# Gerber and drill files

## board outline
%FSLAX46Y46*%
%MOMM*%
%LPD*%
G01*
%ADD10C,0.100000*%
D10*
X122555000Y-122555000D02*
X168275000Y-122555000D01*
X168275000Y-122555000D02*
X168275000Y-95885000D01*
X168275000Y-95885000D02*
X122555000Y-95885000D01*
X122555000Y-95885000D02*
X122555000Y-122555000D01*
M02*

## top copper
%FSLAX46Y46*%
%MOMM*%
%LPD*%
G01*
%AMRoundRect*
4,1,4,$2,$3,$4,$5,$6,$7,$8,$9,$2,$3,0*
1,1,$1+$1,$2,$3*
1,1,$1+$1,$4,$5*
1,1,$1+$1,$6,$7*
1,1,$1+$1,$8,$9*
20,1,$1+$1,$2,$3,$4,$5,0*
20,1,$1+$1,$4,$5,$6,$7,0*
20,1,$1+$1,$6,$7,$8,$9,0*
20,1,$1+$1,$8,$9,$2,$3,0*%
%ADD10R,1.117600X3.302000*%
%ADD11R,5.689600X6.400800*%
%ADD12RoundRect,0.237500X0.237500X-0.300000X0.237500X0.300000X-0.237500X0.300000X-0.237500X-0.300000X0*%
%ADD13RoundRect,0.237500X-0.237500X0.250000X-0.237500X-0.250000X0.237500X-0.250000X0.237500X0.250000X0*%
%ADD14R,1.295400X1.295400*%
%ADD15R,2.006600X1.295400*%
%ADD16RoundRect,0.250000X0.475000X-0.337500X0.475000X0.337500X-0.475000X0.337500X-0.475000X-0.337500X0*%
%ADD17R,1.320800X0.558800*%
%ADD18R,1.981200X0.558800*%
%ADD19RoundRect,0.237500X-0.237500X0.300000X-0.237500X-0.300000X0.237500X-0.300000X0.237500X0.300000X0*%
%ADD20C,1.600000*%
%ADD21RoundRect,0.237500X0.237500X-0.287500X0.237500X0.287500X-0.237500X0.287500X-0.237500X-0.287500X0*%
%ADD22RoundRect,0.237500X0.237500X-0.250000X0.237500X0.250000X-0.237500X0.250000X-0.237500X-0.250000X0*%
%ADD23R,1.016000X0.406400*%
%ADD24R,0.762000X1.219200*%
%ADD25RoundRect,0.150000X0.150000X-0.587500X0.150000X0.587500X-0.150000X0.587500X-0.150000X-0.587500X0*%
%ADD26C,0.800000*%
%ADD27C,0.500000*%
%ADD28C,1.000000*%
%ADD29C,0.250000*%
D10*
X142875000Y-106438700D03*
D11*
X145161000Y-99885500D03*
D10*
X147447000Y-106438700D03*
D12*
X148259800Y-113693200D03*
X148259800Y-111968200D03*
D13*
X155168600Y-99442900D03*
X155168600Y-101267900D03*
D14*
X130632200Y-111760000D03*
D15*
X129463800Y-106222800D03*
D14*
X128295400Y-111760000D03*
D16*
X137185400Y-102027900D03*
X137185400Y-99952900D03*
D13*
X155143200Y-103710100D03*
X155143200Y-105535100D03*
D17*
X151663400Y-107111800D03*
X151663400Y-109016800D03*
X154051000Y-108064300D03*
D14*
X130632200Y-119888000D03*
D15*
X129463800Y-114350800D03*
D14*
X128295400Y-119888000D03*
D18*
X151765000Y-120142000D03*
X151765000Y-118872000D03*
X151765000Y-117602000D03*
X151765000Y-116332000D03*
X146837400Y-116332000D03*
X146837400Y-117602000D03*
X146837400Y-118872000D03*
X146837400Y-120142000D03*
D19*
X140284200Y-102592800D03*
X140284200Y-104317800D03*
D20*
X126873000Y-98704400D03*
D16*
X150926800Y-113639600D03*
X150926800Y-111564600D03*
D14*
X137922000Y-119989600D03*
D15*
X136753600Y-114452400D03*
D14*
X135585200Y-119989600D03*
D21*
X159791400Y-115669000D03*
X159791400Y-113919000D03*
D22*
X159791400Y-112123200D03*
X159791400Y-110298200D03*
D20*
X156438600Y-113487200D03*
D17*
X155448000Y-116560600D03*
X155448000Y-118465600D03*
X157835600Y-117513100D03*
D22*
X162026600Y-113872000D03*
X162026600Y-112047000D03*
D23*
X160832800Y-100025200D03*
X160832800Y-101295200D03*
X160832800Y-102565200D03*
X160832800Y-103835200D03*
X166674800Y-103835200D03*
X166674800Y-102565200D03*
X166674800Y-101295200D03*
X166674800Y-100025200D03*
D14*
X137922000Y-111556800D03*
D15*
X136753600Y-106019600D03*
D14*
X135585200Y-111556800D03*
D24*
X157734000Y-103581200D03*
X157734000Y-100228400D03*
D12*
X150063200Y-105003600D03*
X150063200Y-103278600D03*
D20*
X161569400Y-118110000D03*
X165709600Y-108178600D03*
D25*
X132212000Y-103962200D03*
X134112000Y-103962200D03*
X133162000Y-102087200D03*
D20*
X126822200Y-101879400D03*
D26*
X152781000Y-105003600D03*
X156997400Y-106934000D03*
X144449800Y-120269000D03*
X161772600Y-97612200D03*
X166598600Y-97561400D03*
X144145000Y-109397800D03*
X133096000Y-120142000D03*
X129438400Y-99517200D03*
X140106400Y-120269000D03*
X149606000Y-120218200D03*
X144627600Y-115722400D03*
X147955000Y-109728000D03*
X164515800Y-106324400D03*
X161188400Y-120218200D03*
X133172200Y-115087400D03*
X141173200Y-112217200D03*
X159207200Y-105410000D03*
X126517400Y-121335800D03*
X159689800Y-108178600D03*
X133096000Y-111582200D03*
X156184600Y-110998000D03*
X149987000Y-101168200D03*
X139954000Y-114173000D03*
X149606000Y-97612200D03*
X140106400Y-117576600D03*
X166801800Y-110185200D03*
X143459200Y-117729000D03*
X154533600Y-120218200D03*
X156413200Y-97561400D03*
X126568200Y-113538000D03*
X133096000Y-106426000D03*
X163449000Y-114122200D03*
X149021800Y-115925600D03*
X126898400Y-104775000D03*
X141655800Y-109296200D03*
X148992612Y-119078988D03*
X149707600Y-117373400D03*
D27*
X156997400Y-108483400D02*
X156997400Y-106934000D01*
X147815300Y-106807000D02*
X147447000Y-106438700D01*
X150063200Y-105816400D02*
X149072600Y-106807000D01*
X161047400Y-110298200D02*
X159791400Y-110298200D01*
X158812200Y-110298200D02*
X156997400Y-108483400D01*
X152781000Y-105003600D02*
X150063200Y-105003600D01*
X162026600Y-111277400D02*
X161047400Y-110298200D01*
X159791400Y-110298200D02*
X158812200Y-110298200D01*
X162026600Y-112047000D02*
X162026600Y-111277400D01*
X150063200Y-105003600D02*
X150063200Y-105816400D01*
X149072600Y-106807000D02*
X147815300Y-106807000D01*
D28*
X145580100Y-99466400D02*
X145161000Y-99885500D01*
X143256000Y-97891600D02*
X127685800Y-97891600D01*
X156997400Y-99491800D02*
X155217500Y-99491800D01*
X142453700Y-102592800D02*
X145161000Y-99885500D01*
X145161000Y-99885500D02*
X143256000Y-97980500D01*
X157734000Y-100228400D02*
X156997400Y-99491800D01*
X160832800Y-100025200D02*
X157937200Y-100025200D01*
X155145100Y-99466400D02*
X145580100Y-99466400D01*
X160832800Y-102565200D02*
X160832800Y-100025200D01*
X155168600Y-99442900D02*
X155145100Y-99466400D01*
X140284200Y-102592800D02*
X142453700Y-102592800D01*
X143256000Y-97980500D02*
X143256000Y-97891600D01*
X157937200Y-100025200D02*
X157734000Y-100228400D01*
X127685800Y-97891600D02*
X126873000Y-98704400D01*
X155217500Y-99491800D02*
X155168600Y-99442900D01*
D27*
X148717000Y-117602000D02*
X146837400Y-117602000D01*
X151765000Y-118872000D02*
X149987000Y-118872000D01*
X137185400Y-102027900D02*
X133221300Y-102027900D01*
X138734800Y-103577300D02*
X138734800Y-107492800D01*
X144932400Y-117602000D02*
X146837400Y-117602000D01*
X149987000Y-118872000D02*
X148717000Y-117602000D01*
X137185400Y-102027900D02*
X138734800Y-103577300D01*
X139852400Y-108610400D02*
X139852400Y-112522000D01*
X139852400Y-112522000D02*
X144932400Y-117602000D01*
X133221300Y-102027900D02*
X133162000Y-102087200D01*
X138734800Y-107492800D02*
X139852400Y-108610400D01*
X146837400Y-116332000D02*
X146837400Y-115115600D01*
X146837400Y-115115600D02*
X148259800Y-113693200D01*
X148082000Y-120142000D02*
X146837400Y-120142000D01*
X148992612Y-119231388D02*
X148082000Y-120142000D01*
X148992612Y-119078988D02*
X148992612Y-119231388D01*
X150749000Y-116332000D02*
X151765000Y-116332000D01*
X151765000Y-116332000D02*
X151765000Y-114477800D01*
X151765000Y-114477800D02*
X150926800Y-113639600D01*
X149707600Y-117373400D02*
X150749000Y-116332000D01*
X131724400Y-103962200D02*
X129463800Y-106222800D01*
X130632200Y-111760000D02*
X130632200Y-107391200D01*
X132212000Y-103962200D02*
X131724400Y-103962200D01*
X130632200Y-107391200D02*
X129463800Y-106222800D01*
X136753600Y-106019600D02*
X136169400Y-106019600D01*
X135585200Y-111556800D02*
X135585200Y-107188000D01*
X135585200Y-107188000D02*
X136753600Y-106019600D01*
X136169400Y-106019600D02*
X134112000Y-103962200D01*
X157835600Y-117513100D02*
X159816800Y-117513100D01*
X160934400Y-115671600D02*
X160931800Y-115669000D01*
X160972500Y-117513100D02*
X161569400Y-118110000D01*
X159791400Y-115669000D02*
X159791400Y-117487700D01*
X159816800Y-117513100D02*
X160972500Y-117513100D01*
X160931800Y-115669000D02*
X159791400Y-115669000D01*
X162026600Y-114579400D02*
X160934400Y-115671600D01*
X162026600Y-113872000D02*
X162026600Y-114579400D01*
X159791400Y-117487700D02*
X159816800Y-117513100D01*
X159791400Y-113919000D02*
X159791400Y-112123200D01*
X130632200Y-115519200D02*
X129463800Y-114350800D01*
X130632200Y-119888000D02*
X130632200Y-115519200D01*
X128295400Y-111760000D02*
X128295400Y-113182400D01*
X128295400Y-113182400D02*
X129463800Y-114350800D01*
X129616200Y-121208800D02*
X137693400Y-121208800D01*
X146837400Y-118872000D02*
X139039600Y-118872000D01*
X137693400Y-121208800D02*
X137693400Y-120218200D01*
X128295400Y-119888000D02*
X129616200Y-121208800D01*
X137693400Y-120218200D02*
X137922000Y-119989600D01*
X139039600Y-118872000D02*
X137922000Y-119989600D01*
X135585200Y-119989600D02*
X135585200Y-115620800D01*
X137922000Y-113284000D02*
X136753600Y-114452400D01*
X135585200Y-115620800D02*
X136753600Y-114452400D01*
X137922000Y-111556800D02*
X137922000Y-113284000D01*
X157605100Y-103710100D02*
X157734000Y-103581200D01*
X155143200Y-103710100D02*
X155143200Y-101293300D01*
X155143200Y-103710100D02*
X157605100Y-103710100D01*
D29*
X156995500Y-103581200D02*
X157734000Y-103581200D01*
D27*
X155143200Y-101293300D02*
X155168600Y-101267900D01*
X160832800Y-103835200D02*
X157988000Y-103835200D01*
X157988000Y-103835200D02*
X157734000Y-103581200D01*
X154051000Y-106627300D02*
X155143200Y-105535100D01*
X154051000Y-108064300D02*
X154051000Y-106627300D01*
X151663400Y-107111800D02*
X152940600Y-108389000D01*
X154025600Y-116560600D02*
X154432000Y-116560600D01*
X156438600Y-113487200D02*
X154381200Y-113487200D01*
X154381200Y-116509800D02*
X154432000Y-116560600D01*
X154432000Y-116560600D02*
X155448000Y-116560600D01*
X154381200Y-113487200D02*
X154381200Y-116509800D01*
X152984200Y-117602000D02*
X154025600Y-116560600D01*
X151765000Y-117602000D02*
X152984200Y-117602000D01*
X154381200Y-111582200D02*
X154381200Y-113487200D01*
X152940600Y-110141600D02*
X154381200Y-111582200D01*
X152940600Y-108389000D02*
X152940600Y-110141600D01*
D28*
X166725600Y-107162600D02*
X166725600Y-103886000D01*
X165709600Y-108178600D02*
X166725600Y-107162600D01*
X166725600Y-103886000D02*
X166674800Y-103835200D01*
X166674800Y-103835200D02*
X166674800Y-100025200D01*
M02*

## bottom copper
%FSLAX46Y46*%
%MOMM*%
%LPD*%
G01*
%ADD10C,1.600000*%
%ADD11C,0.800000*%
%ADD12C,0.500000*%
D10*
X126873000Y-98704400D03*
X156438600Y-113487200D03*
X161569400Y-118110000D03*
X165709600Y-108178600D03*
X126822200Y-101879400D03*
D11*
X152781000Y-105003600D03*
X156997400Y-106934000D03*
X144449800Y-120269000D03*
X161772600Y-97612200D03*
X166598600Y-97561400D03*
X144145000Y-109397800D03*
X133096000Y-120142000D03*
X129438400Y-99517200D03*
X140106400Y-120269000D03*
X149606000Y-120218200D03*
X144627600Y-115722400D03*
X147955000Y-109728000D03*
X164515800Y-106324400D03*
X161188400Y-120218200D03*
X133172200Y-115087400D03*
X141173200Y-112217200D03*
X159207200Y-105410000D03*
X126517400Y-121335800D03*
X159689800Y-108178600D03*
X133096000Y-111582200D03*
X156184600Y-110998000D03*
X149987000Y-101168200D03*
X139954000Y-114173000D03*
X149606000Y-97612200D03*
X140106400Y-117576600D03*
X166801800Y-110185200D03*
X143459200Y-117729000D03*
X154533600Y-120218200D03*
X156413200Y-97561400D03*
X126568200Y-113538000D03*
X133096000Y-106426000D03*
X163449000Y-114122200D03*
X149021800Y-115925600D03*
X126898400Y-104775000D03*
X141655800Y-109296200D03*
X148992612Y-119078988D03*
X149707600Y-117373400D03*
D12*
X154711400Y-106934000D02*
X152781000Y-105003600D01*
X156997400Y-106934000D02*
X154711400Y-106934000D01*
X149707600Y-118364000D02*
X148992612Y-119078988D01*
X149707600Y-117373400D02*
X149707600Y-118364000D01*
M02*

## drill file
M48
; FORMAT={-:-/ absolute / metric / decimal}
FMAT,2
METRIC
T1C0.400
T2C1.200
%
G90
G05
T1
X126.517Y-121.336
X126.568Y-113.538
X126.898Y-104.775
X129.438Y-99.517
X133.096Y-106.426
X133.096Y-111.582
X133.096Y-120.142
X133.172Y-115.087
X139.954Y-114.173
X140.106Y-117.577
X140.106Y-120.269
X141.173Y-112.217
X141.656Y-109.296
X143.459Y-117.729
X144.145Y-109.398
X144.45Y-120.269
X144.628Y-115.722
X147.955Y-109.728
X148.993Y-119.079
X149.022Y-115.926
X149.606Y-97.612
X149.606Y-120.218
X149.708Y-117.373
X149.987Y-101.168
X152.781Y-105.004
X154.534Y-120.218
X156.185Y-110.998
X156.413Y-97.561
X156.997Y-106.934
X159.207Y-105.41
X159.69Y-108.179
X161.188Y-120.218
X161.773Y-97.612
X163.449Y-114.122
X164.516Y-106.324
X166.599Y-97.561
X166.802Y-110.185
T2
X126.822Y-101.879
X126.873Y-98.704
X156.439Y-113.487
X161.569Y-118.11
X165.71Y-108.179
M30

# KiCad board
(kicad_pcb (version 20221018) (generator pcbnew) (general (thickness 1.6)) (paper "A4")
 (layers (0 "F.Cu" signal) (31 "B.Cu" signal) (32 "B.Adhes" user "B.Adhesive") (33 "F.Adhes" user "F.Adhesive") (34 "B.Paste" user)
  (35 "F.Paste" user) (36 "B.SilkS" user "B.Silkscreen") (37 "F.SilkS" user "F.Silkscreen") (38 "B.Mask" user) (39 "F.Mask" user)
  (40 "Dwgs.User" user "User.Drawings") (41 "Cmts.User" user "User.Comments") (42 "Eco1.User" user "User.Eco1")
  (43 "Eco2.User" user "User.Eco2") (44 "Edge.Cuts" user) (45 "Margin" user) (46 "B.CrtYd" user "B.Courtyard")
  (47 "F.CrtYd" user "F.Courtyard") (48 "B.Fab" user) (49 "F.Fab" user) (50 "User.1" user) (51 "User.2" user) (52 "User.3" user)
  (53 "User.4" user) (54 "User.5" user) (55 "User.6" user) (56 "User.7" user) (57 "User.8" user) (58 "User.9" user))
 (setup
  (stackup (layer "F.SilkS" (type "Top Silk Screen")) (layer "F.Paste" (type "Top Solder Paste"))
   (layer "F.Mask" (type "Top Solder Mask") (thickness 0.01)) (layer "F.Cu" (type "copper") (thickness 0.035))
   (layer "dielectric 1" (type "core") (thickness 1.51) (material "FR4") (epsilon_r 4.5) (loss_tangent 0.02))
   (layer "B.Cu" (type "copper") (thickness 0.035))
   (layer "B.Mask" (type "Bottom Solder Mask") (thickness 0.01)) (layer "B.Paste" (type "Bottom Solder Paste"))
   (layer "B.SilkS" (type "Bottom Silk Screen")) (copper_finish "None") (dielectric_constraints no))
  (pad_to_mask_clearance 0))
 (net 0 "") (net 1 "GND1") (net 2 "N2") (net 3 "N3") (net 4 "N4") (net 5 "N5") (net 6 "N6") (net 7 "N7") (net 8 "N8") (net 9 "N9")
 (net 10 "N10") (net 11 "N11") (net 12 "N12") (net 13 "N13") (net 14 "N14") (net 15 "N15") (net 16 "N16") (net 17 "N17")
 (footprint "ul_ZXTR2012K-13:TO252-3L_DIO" (layer "F.Cu") (at 145.161 99.8855)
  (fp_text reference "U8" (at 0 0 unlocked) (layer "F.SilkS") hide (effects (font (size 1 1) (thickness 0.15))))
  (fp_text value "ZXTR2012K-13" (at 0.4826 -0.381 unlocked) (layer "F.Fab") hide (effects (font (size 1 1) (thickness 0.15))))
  (pad "1" smd rect (at -2.286 6.5532) (size 1.1176 3.302) (layers "F.Cu" "F.Paste" "F.Mask") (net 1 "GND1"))
  (pad "2" smd rect (at 0 0) (size 5.6896 6.4008) (layers "F.Cu" "F.Paste" "F.Mask") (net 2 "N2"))
  (pad "3" smd rect (at 2.286 6.5532) (size 1.1176 3.302) (layers "F.Cu" "F.Paste" "F.Mask") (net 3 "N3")))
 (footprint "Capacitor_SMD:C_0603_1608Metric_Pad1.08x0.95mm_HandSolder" (layer "F.Cu") (at 148.2598 112.8307 90)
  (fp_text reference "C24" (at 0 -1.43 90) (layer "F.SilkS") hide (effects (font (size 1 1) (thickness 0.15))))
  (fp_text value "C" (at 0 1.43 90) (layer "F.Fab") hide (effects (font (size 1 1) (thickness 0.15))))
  (pad "1" smd roundrect (at -0.8625 0 90) (size 1.075 0.95) (layers "F.Cu" "F.Paste" "F.Mask") (roundrect_rratio 0.25) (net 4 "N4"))
  (pad "2" smd roundrect (at 0.8625 0 90) (size 1.075 0.95) (layers "F.Cu" "F.Paste" "F.Mask") (roundrect_rratio 0.25) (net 1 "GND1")))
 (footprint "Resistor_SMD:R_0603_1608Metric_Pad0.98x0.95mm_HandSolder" (layer "F.Cu") (at 155.1686 100.3554 -90)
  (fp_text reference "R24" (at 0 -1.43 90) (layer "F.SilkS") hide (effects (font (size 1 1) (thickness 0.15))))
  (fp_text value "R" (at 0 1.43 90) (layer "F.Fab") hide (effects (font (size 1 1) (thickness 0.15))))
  (pad "1" smd roundrect (at -0.9125 0 270) (size 0.975 0.95) (layers "F.Cu" "F.Paste" "F.Mask") (roundrect_rratio 0.25) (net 2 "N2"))
  (pad "2" smd roundrect (at 0.9125 0 270) (size 0.975 0.95) (layers "F.Cu" "F.Paste" "F.Mask") (roundrect_rratio 0.25) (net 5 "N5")))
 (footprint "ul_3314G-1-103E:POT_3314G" (layer "F.Cu") (at 129.4638 108.9914)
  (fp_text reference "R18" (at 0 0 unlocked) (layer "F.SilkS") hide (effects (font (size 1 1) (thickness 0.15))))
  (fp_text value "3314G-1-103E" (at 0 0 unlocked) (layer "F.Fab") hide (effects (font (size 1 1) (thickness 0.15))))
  (pad "1" smd rect (at 1.1684 2.7686) (size 1.2954 1.2954) (layers "F.Cu" "F.Paste" "F.Mask") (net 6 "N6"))
  (pad "2" smd rect (at 0 -2.7686) (size 2.0066 1.2954) (layers "F.Cu" "F.Paste" "F.Mask") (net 6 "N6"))
  (pad "3" smd rect (at -1.1684 2.7686) (size 1.2954 1.2954) (layers "F.Cu" "F.Paste" "F.Mask") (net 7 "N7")))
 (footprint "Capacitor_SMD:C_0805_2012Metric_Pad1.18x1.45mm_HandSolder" (layer "F.Cu") (at 137.1854 100.9904 90)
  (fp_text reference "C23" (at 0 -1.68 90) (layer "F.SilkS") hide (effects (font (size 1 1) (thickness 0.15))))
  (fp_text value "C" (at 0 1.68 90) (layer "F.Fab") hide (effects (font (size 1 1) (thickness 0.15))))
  (pad "1" smd roundrect (at -1.0375 0 90) (size 1.175 1.45) (layers "F.Cu" "F.Paste" "F.Mask") (roundrect_rratio 0.212766) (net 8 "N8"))
  (pad "2" smd roundrect (at 1.0375 0 90) (size 1.175 1.45) (layers "F.Cu" "F.Paste" "F.Mask") (roundrect_rratio 0.212766) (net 1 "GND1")))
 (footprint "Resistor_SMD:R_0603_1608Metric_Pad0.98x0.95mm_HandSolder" (layer "F.Cu") (at 155.1432 104.6226 -90)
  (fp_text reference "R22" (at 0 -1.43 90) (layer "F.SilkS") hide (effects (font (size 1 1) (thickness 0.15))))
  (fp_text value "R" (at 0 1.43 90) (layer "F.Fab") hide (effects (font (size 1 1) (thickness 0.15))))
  (pad "1" smd roundrect (at -0.9125 0 270) (size 0.975 0.95) (layers "F.Cu" "F.Paste" "F.Mask") (roundrect_rratio 0.25) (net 5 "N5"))
  (pad "2" smd roundrect (at 0.9125 0 270) (size 0.975 0.95) (layers "F.Cu" "F.Paste" "F.Mask") (roundrect_rratio 0.25) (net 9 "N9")))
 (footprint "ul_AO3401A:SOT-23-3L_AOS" (layer "F.Cu") (at 152.8572 108.0643 -90)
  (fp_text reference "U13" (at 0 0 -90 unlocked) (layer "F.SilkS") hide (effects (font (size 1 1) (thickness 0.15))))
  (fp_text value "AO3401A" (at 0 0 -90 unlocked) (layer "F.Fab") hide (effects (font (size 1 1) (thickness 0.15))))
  (pad "1" smd rect (at -0.9525 1.1938 270) (size 0.5588 1.3208) (layers "F.Cu" "F.Paste" "F.Mask") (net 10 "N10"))
  (pad "2" smd rect (at 0.9525 1.1938 270) (size 0.5588 1.3208) (layers "F.Cu" "F.Paste" "F.Mask") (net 1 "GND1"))
  (pad "3" smd rect (at 0 -1.1938 270) (size 0.5588 1.3208) (layers "F.Cu" "F.Paste" "F.Mask") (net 9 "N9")))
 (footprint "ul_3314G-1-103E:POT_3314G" (layer "F.Cu") (at 129.4638 117.1194)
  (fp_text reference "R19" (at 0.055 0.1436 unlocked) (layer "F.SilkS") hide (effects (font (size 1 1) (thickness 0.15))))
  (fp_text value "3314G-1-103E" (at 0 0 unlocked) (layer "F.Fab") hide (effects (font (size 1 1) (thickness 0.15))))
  (pad "1" smd rect (at 1.1684 2.7686) (size 1.2954 1.2954) (layers "F.Cu" "F.Paste" "F.Mask") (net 7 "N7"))
  (pad "2" smd rect (at 0 -2.7686) (size 2.0066 1.2954) (layers "F.Cu" "F.Paste" "F.Mask") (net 7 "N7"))
  (pad "3" smd rect (at -1.1684 2.7686) (size 1.2954 1.2954) (layers "F.Cu" "F.Paste" "F.Mask") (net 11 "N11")))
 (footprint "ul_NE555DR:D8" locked (layer "F.Cu") (at 149.3012 118.237 180)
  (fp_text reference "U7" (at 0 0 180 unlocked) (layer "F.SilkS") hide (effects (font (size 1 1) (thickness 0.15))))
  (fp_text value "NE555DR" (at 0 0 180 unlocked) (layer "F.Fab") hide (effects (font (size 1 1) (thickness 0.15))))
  (pad "1" smd rect locked (at -2.4638 -1.905 180) (size 1.9812 0.5588) (layers "F.Cu" "F.Paste" "F.Mask") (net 1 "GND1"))
  (pad "2" smd rect locked (at -2.4638 -0.635 180) (size 1.9812 0.5588) (layers "F.Cu" "F.Paste" "F.Mask") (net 8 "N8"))
  (pad "3" smd rect locked (at -2.4638 0.635 180) (size 1.9812 0.5588) (layers "F.Cu" "F.Paste" "F.Mask") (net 10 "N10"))
  (pad "4" smd rect locked (at -2.4638 1.905 180) (size 1.9812 0.5588) (layers "F.Cu" "F.Paste" "F.Mask") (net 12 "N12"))
  (pad "5" smd rect locked (at 2.4638 1.905 180) (size 1.9812 0.5588) (layers "F.Cu" "F.Paste" "F.Mask") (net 4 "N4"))
  (pad "6" smd rect locked (at 2.4638 0.635 180) (size 1.9812 0.5588) (layers "F.Cu" "F.Paste" "F.Mask") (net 8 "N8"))
  (pad "7" smd rect locked (at 2.4638 -0.635 180) (size 1.9812 0.5588) (layers "F.Cu" "F.Paste" "F.Mask") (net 11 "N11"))
  (pad "8" smd rect locked (at 2.4638 -1.905 180) (size 1.9812 0.5588) (layers "F.Cu" "F.Paste" "F.Mask") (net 12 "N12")))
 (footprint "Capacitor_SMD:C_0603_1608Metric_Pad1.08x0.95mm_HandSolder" (layer "F.Cu") (at 140.2842 103.4553 -90)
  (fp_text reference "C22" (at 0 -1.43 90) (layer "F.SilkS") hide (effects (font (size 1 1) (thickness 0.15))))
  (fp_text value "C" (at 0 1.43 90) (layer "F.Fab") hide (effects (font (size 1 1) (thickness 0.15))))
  (pad "1" smd roundrect (at -0.8625 0 270) (size 1.075 0.95) (layers "F.Cu" "F.Paste" "F.Mask") (roundrect_rratio 0.25) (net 2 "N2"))
  (pad "2" smd roundrect (at 0.8625 0 270) (size 1.075 0.95) (layers "F.Cu" "F.Paste" "F.Mask") (roundrect_rratio 0.25) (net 1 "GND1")))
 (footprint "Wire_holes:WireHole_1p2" (layer "F.Cu") (at 126.873 98.7044)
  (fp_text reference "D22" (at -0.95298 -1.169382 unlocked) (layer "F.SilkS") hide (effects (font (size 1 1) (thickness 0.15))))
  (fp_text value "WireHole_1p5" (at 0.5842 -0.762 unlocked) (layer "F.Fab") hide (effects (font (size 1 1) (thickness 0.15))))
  (pad "1" thru_hole circle (at 0 0) (size 1.6 1.6) (drill 1.2) (layers "*.Cu" "*.Mask") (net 2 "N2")))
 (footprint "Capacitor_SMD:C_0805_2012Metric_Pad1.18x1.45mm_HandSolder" (layer "F.Cu") (at 150.9268 112.6021 90)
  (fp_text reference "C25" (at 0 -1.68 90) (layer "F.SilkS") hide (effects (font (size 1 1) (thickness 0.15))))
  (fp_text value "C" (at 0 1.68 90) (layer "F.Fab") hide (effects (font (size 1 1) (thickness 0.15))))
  (pad "1" smd roundrect (at -1.0375 0 90) (size 1.175 1.45) (layers "F.Cu" "F.Paste" "F.Mask") (roundrect_rratio 0.212766) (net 12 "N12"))
  (pad "2" smd roundrect (at 1.0375 0 90) (size 1.175 1.45) (layers "F.Cu" "F.Paste" "F.Mask") (roundrect_rratio 0.212766) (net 1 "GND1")))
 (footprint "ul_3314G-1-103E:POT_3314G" (layer "F.Cu") (at 136.7536 117.221)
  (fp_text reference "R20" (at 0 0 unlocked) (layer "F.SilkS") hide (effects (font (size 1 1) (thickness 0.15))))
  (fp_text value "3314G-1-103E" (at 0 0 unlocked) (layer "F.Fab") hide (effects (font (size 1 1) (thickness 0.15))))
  (pad "1" smd rect (at 1.1684 2.7686) (size 1.2954 1.2954) (layers "F.Cu" "F.Paste" "F.Mask") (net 11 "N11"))
  (pad "2" smd rect (at 0 -2.7686) (size 2.0066 1.2954) (layers "F.Cu" "F.Paste" "F.Mask") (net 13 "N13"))
  (pad "3" smd rect (at -1.1684 2.7686) (size 1.2954 1.2954) (layers "F.Cu" "F.Paste" "F.Mask") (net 13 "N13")))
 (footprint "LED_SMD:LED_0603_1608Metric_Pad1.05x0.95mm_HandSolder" (layer "F.Cu") (at 159.7914 114.794 90)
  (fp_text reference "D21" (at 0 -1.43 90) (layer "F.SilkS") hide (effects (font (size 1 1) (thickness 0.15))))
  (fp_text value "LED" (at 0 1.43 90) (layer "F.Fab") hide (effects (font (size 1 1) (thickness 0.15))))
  (pad "1" smd roundrect (at -0.875 0 90) (size 1.05 0.95) (layers "F.Cu" "F.Paste" "F.Mask") (roundrect_rratio 0.25) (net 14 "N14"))
  (pad "2" smd roundrect (at 0.875 0 90) (size 1.05 0.95) (layers "F.Cu" "F.Paste" "F.Mask") (roundrect_rratio 0.25) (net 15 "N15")))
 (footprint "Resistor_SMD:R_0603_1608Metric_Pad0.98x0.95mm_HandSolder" (layer "F.Cu") (at 159.7914 111.2107 90)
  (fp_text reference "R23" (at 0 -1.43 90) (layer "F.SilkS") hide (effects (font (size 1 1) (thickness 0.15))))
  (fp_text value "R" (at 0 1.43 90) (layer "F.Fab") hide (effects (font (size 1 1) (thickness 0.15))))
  (pad "1" smd roundrect (at -0.9125 0 90) (size 0.975 0.95) (layers "F.Cu" "F.Paste" "F.Mask") (roundrect_rratio 0.25) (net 15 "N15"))
  (pad "2" smd roundrect (at 0.9125 0 90) (size 0.975 0.95) (layers "F.Cu" "F.Paste" "F.Mask") (roundrect_rratio 0.25) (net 3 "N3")))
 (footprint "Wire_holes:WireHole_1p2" (layer "F.Cu") (at 156.4386 113.4872)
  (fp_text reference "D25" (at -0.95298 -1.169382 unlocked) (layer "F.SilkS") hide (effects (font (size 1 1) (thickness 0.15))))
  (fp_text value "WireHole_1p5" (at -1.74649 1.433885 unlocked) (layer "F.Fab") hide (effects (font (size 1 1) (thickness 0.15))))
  (pad "1" thru_hole circle (at 0 0) (size 1.6 1.6) (drill 1.2) (layers "*.Cu" "*.Mask") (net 10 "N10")))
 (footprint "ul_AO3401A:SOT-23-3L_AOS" (layer "F.Cu") (at 156.6418 117.5131 -90)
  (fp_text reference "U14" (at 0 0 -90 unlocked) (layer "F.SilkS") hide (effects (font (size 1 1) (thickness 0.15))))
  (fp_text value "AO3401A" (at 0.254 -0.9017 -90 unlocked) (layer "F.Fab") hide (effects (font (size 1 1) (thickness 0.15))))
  (pad "1" smd rect (at -0.9525 1.1938 270) (size 0.5588 1.3208) (layers "F.Cu" "F.Paste" "F.Mask") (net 10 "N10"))
  (pad "2" smd rect (at 0.9525 1.1938 270) (size 0.5588 1.3208) (layers "F.Cu" "F.Paste" "F.Mask") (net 1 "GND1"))
  (pad "3" smd rect (at 0 -1.1938 270) (size 0.5588 1.3208) (layers "F.Cu" "F.Paste" "F.Mask") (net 14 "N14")))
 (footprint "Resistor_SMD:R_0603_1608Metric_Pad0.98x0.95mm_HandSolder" (layer "F.Cu") (at 162.0266 112.9595 90)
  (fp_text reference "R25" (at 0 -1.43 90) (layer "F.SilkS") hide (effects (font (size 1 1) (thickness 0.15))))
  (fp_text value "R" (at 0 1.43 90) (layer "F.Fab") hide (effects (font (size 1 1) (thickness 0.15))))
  (pad "1" smd roundrect (at -0.9125 0 90) (size 0.975 0.95) (layers "F.Cu" "F.Paste" "F.Mask") (roundrect_rratio 0.25) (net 14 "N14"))
  (pad "2" smd roundrect (at 0.9125 0 90) (size 0.975 0.95) (layers "F.Cu" "F.Paste" "F.Mask") (roundrect_rratio 0.25) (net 3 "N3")))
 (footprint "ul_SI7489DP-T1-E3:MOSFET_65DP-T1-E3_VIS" (layer "F.Cu") (at 163.7538 101.9302)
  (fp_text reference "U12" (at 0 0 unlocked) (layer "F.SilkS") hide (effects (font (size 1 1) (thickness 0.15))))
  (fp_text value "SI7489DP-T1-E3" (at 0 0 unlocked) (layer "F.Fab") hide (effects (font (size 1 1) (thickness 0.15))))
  (pad "1" smd rect (at -2.921 -1.905) (size 1.016 0.4064) (layers "F.Cu" "F.Paste" "F.Mask") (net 2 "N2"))
  (pad "2" smd rect (at -2.921 -0.635) (size 1.016 0.4064) (layers "F.Cu" "F.Paste" "F.Mask") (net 2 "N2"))
  (pad "3" smd rect (at -2.921 0.635) (size 1.016 0.4064) (layers "F.Cu" "F.Paste" "F.Mask") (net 2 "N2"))
  (pad "4" smd rect (at -2.921 1.905) (size 1.016 0.4064) (layers "F.Cu" "F.Paste" "F.Mask") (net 5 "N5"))
  (pad "5" smd rect (at 2.921 1.905) (size 1.016 0.4064) (layers "F.Cu" "F.Paste" "F.Mask") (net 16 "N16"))
  (pad "6" smd rect (at 2.921 0.635) (size 1.016 0.4064) (layers "F.Cu" "F.Paste" "F.Mask") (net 16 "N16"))
  (pad "7" smd rect (at 2.921 -0.635) (size 1.016 0.4064) (layers "F.Cu" "F.Paste" "F.Mask") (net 16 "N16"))
  (pad "8" smd rect (at 2.921 -1.905) (size 1.016 0.4064) (layers "F.Cu" "F.Paste" "F.Mask") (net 16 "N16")))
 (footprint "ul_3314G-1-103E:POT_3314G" (layer "F.Cu") (at 136.7536 108.7882)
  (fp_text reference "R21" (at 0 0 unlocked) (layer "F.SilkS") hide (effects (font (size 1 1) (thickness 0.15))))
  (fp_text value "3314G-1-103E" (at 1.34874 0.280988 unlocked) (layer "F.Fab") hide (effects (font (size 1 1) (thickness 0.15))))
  (pad "1" smd rect (at 1.1684 2.7686) (size 1.2954 1.2954) (layers "F.Cu" "F.Paste" "F.Mask") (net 13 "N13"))
  (pad "2" smd rect (at 0 -2.7686) (size 2.0066 1.2954) (layers "F.Cu" "F.Paste" "F.Mask") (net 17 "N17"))
  (pad "3" smd rect (at -1.1684 2.7686) (size 1.2954 1.2954) (layers "F.Cu" "F.Paste" "F.Mask") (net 17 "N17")))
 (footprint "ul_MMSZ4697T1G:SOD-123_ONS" (layer "F.Cu") (at 157.734 101.9048 90)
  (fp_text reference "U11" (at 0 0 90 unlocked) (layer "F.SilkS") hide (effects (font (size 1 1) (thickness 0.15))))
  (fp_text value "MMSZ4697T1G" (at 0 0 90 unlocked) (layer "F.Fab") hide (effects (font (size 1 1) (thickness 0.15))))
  (pad "1" smd rect (at -1.6764 0 90) (size 1.2192 0.762) (layers "F.Cu" "F.Paste" "F.Mask") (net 5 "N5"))
  (pad "2" smd rect (at 1.6764 0 90) (size 1.2192 0.762) (layers "F.Cu" "F.Paste" "F.Mask") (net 2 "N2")))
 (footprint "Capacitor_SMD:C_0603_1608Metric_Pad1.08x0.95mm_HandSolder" (layer "F.Cu") (at 150.0632 104.1411 90)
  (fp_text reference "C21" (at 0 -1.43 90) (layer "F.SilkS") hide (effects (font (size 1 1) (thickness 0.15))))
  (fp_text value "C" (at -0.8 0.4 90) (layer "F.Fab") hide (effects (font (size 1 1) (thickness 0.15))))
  (pad "1" smd roundrect (at -0.8625 0 90) (size 1.075 0.95) (layers "F.Cu" "F.Paste" "F.Mask") (roundrect_rratio 0.25) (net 3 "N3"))
  (pad "2" smd roundrect (at 0.8625 0 90) (size 1.075 0.95) (layers "F.Cu" "F.Paste" "F.Mask") (roundrect_rratio 0.25) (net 1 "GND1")))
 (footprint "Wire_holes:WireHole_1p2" (layer "F.Cu") (at 161.5694 118.11)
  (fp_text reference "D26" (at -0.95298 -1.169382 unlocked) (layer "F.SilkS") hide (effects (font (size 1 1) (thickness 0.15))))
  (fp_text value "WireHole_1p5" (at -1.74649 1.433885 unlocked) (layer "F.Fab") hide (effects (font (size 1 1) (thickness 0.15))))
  (pad "1" thru_hole circle (at 0 0) (size 1.6 1.6) (drill 1.2) (layers "*.Cu" "*.Mask") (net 14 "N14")))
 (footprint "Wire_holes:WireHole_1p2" (layer "F.Cu") (at 165.7096 108.1786)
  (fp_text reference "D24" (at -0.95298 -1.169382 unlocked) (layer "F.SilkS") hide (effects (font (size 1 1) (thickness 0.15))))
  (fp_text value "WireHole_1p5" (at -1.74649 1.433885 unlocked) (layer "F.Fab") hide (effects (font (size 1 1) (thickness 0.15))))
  (pad "1" thru_hole circle (at 0 0) (size 1.6 1.6) (drill 1.2) (layers "*.Cu" "*.Mask") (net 16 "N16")))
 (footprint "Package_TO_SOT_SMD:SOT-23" (layer "F.Cu") (at 133.162 103.0247 90)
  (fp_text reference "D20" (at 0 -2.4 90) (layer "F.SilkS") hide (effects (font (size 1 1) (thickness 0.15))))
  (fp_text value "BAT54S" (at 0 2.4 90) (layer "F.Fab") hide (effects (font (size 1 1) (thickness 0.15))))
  (pad "1" smd roundrect (at -0.9375 -0.95 90) (size 1.475 0.6) (layers "F.Cu" "F.Paste" "F.Mask") (roundrect_rratio 0.25) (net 6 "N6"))
  (pad "2" smd roundrect (at -0.9375 0.95 90) (size 1.475 0.6) (layers "F.Cu" "F.Paste" "F.Mask") (roundrect_rratio 0.25) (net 17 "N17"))
  (pad "3" smd roundrect (at 0.9375 0 90) (size 1.475 0.6) (layers "F.Cu" "F.Paste" "F.Mask") (roundrect_rratio 0.25) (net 8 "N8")))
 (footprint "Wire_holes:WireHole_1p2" (layer "F.Cu") (at 126.8222 101.8794)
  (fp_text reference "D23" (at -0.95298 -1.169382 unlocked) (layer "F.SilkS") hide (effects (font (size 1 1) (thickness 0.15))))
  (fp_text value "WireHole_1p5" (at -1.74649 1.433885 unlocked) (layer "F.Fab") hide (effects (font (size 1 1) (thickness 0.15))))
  (pad "1" thru_hole circle (at 0 0) (size 1.6 1.6) (drill 1.2) (layers "*.Cu" "*.Mask") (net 1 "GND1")))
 (gr_line (start 122.555 122.555) (end 168.275 122.555) (stroke (width 0.1) (type default)) (layer "Edge.Cuts"))
 (gr_line (start 168.275 122.555) (end 168.275 95.885) (stroke (width 0.1) (type default)) (layer "Edge.Cuts"))
 (gr_line (start 168.275 95.885) (end 122.555 95.885) (stroke (width 0.1) (type default)) (layer "Edge.Cuts"))
 (gr_line (start 122.555 95.885) (end 122.555 122.555) (stroke (width 0.1) (type default)) (layer "Edge.Cuts"))
 (segment (start 156.9974 108.4834) (end 156.9974 106.934) (width 0.5) (layer "F.Cu") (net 3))
 (segment (start 147.8153 106.807) (end 147.447 106.4387) (width 0.5) (layer "F.Cu") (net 3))
 (segment (start 150.0632 105.8164) (end 149.0726 106.807) (width 0.5) (layer "F.Cu") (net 3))
 (segment (start 161.0474 110.2982) (end 159.7914 110.2982) (width 0.5) (layer "F.Cu") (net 3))
 (segment (start 158.8122 110.2982) (end 156.9974 108.4834) (width 0.5) (layer "F.Cu") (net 3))
 (segment (start 152.781 105.0036) (end 150.0632 105.0036) (width 0.5) (layer "F.Cu") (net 3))
 (segment (start 162.0266 111.2774) (end 161.0474 110.2982) (width 0.5) (layer "F.Cu") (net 3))
 (segment (start 159.7914 110.2982) (end 158.8122 110.2982) (width 0.5) (layer "F.Cu") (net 3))
 (segment (start 162.0266 112.047) (end 162.0266 111.2774) (width 0.5) (layer "F.Cu") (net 3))
 (segment (start 150.0632 105.0036) (end 150.0632 105.8164) (width 0.5) (layer "F.Cu") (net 3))
 (segment (start 149.0726 106.807) (end 147.8153 106.807) (width 0.5) (layer "F.Cu") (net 3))
 (via (at 152.781 105.0036) (size 0.8) (drill 0.4) (layers "F.Cu" "B.Cu") (free) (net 3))
 (via (at 156.9974 106.934) (size 0.8) (drill 0.4) (layers "F.Cu" "B.Cu") (free) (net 3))
 (segment (start 154.7114 106.934) (end 152.781 105.0036) (width 0.5) (layer "B.Cu") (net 3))
 (segment (start 156.9974 106.934) (end 154.7114 106.934) (width 0.5) (layer "B.Cu") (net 3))
 (via (at 144.4498 120.269) (size 0.8) (drill 0.4) (layers "F.Cu" "B.Cu") (free) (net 1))
 (via (at 161.7726 97.6122) (size 0.8) (drill 0.4) (layers "F.Cu" "B.Cu") (free) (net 1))
 (via (at 166.5986 97.5614) (size 0.8) (drill 0.4) (layers "F.Cu" "B.Cu") (free) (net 1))
 (via (at 144.145 109.3978) (size 0.8) (drill 0.4) (layers "F.Cu" "B.Cu") (free) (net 1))
 (via (at 133.096 120.142) (size 0.8) (drill 0.4) (layers "F.Cu" "B.Cu") (free) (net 1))
 (via (at 129.4384 99.5172) (size 0.8) (drill 0.4) (layers "F.Cu" "B.Cu") (free) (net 1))
 (via (at 140.1064 120.269) (size 0.8) (drill 0.4) (layers "F.Cu" "B.Cu") (free) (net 1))
 (via (at 149.606 120.2182) (size 0.8) (drill 0.4) (layers "F.Cu" "B.Cu") (free) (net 1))
 (via (at 144.6276 115.7224) (size 0.8) (drill 0.4) (layers "F.Cu" "B.Cu") (free) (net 1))
 (via (at 147.955 109.728) (size 0.8) (drill 0.4) (layers "F.Cu" "B.Cu") (free) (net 1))
 (via (at 164.5158 106.3244) (size 0.8) (drill 0.4) (layers "F.Cu" "B.Cu") (free) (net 1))
 (via (at 161.1884 120.2182) (size 0.8) (drill 0.4) (layers "F.Cu" "B.Cu") (free) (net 1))
 (via (at 133.1722 115.0874) (size 0.8) (drill 0.4) (layers "F.Cu" "B.Cu") (free) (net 1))
 (via (at 141.1732 112.2172) (size 0.8) (drill 0.4) (layers "F.Cu" "B.Cu") (free) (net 1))
 (via (at 159.2072 105.41) (size 0.8) (drill 0.4) (layers "F.Cu" "B.Cu") (free) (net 1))
 (via (at 126.5174 121.3358) (size 0.8) (drill 0.4) (layers "F.Cu" "B.Cu") (free) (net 1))
 (via (at 159.6898 108.1786) (size 0.8) (drill 0.4) (layers "F.Cu" "B.Cu") (free) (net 1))
 (via (at 133.096 111.5822) (size 0.8) (drill 0.4) (layers "F.Cu" "B.Cu") (free) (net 1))
 (via (at 156.1846 110.998) (size 0.8) (drill 0.4) (layers "F.Cu" "B.Cu") (free) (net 1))
 (via (at 149.987 101.1682) (size 0.8) (drill 0.4) (layers "F.Cu" "B.Cu") (free) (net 1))
 (via (at 139.954 114.173) (size 0.8) (drill 0.4) (layers "F.Cu" "B.Cu") (free) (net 1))
 (via (at 149.606 97.6122) (size 0.8) (drill 0.4) (layers "F.Cu" "B.Cu") (free) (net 1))
 (via (at 140.1064 117.5766) (size 0.8) (drill 0.4) (layers "F.Cu" "B.Cu") (free) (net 1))
 (via (at 166.8018 110.1852) (size 0.8) (drill 0.4) (layers "F.Cu" "B.Cu") (free) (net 1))
 (via (at 143.4592 117.729) (size 0.8) (drill 0.4) (layers "F.Cu" "B.Cu") (free) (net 1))
 (via (at 154.5336 120.2182) (size 0.8) (drill 0.4) (layers "F.Cu" "B.Cu") (free) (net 1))
 (via (at 156.4132 97.5614) (size 0.8) (drill 0.4) (layers "F.Cu" "B.Cu") (free) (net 1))
 (via (at 126.5682 113.538) (size 0.8) (drill 0.4) (layers "F.Cu" "B.Cu") (free) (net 1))
 (via (at 133.096 106.426) (size 0.8) (drill 0.4) (layers "F.Cu" "B.Cu") (free) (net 1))
 (via (at 163.449 114.1222) (size 0.8) (drill 0.4) (layers "F.Cu" "B.Cu") (free) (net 1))
 (via (at 149.0218 115.9256) (size 0.8) (drill 0.4) (layers "F.Cu" "B.Cu") (free) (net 1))
 (via (at 126.8984 104.775) (size 0.8) (drill 0.4) (layers "F.Cu" "B.Cu") (free) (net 1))
 (via (at 141.6558 109.2962) (size 0.8) (drill 0.4) (layers "F.Cu" "B.Cu") (free) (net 1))
 (segment (start 145.5801 99.4664) (end 145.161 99.8855) (width 1) (layer "F.Cu") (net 2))
 (segment (start 143.256 97.8916) (end 127.6858 97.8916) (width 1) (layer "F.Cu") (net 2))
 (segment (start 156.9974 99.4918) (end 155.2175 99.4918) (width 1) (layer "F.Cu") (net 2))
 (segment (start 142.4537 102.5928) (end 145.161 99.8855) (width 1) (layer "F.Cu") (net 2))
 (segment (start 145.161 99.8855) (end 143.256 97.9805) (width 1) (layer "F.Cu") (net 2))
 (segment (start 157.734 100.2284) (end 156.9974 99.4918) (width 1) (layer "F.Cu") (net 2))
 (segment (start 160.8328 100.0252) (end 157.9372 100.0252) (width 1) (layer "F.Cu") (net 2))
 (segment (start 155.1451 99.4664) (end 145.5801 99.4664) (width 1) (layer "F.Cu") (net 2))
 (segment (start 160.8328 102.5652) (end 160.8328 100.0252) (width 1) (layer "F.Cu") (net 2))
 (segment (start 155.1686 99.4429) (end 155.1451 99.4664) (width 1) (layer "F.Cu") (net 2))
 (segment (start 140.2842 102.5928) (end 142.4537 102.5928) (width 1) (layer "F.Cu") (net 2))
 (segment (start 143.256 97.9805) (end 143.256 97.8916) (width 1) (layer "F.Cu") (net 2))
 (segment (start 157.9372 100.0252) (end 157.734 100.2284) (width 1) (layer "F.Cu") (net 2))
 (segment (start 127.6858 97.8916) (end 126.873 98.7044) (width 1) (layer "F.Cu") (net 2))
 (segment (start 155.2175 99.4918) (end 155.1686 99.4429) (width 1) (layer "F.Cu") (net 2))
 (segment (start 148.717 117.602) (end 146.8374 117.602) (width 0.5) (layer "F.Cu") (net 8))
 (segment (start 151.765 118.872) (end 149.987 118.872) (width 0.5) (layer "F.Cu") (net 8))
 (segment (start 137.1854 102.0279) (end 133.2213 102.0279) (width 0.5) (layer "F.Cu") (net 8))
 (segment (start 138.7348 103.5773) (end 138.7348 107.4928) (width 0.5) (layer "F.Cu") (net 8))
 (segment (start 144.9324 117.602) (end 146.8374 117.602) (width 0.5) (layer "F.Cu") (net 8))
 (segment (start 149.987 118.872) (end 148.717 117.602) (width 0.5) (layer "F.Cu") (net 8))
 (segment (start 137.1854 102.0279) (end 138.7348 103.5773) (width 0.5) (layer "F.Cu") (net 8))
 (segment (start 139.8524 108.6104) (end 139.8524 112.522) (width 0.5) (layer "F.Cu") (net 8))
 (segment (start 139.8524 112.522) (end 144.9324 117.602) (width 0.5) (layer "F.Cu") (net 8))
 (segment (start 133.2213 102.0279) (end 133.162 102.0872) (width 0.5) (layer "F.Cu") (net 8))
 (segment (start 138.7348 107.4928) (end 139.8524 108.6104) (width 0.5) (layer "F.Cu") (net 8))
 (segment (start 146.8374 116.332) (end 146.8374 115.1156) (width 0.5) (layer "F.Cu") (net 4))
 (segment (start 146.8374 115.1156) (end 148.2598 113.6932) (width 0.5) (layer "F.Cu") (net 4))
 (segment (start 148.082 120.142) (end 146.8374 120.142) (width 0.5) (layer "F.Cu") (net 12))
 (segment (start 148.992612 119.231388) (end 148.082 120.142) (width 0.5) (layer "F.Cu") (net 12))
 (segment (start 148.992612 119.078988) (end 148.992612 119.231388) (width 0.5) (layer "F.Cu") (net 12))
 (segment (start 150.749 116.332) (end 151.765 116.332) (width 0.5) (layer "F.Cu") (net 12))
 (segment (start 151.765 116.332) (end 151.765 114.4778) (width 0.5) (layer "F.Cu") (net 12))
 (segment (start 151.765 114.4778) (end 150.9268 113.6396) (width 0.5) (layer "F.Cu") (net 12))
 (segment (start 149.7076 117.3734) (end 150.749 116.332) (width 0.5) (layer "F.Cu") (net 12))
 (via (at 148.992612 119.078988) (size 0.8) (drill 0.4) (layers "F.Cu" "B.Cu") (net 12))
 (via (at 149.7076 117.3734) (size 0.8) (drill 0.4) (layers "F.Cu" "B.Cu") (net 12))
 (segment (start 149.7076 118.364) (end 148.992612 119.078988) (width 0.5) (layer "B.Cu") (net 12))
 (segment (start 149.7076 117.3734) (end 149.7076 118.364) (width 0.5) (layer "B.Cu") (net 12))
 (segment (start 131.7244 103.9622) (end 129.4638 106.2228) (width 0.5) (layer "F.Cu") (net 6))
 (segment (start 130.6322 111.76) (end 130.6322 107.3912) (width 0.5) (layer "F.Cu") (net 6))
 (segment (start 132.212 103.9622) (end 131.7244 103.9622) (width 0.5) (layer "F.Cu") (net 6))
 (segment (start 130.6322 107.3912) (end 129.4638 106.2228) (width 0.5) (layer "F.Cu") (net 6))
 (segment (start 136.7536 106.0196) (end 136.1694 106.0196) (width 0.5) (layer "F.Cu") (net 17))
 (segment (start 135.5852 111.5568) (end 135.5852 107.188) (width 0.5) (layer "F.Cu") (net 17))
 (segment (start 135.5852 107.188) (end 136.7536 106.0196) (width 0.5) (layer "F.Cu") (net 17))
 (segment (start 136.1694 106.0196) (end 134.112 103.9622) (width 0.5) (layer "F.Cu") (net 17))
 (segment (start 157.8356 117.5131) (end 159.8168 117.5131) (width 0.5) (layer "F.Cu") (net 14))
 (segment (start 160.9344 115.6716) (end 160.9318 115.669) (width 0.5) (layer "F.Cu") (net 14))
 (segment (start 160.9725 117.5131) (end 161.5694 118.11) (width 0.5) (layer "F.Cu") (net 14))
 (segment (start 159.7914 115.669) (end 159.7914 117.4877) (width 0.5) (layer "F.Cu") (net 14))
 (segment (start 159.8168 117.5131) (end 160.9725 117.5131) (width 0.5) (layer "F.Cu") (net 14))
 (segment (start 160.9318 115.669) (end 159.7914 115.669) (width 0.5) (layer "F.Cu") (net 14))
 (segment (start 162.0266 114.5794) (end 160.9344 115.6716) (width 0.5) (layer "F.Cu") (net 14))
 (segment (start 162.0266 113.872) (end 162.0266 114.5794) (width 0.5) (layer "F.Cu") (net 14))
 (segment (start 159.7914 117.4877) (end 159.8168 117.5131) (width 0.5) (layer "F.Cu") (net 14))
 (segment (start 159.7914 113.919) (end 159.7914 112.1232) (width 0.5) (layer "F.Cu") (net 15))
 (segment (start 130.6322 115.5192) (end 129.4638 114.3508) (width 0.5) (layer "F.Cu") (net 7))
 (segment (start 130.6322 119.888) (end 130.6322 115.5192) (width 0.5) (layer "F.Cu") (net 7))
 (segment (start 128.2954 111.76) (end 128.2954 113.1824) (width 0.5) (layer "F.Cu") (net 7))
 (segment (start 128.2954 113.1824) (end 129.4638 114.3508) (width 0.5) (layer "F.Cu") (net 7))
 (segment (start 129.6162 121.2088) (end 137.6934 121.2088) (width 0.5) (layer "F.Cu") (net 11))
 (segment (start 146.8374 118.872) (end 139.0396 118.872) (width 0.5) (layer "F.Cu") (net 11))
 (segment (start 137.6934 121.2088) (end 137.6934 120.2182) (width 0.5) (layer "F.Cu") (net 11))
 (segment (start 128.2954 119.888) (end 129.6162 121.2088) (width 0.5) (layer "F.Cu") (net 11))
 (segment (start 137.6934 120.2182) (end 137.922 119.9896) (width 0.5) (layer "F.Cu") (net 11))
 (segment (start 139.0396 118.872) (end 137.922 119.9896) (width 0.5) (layer "F.Cu") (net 11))
 (segment (start 135.5852 119.9896) (end 135.5852 115.6208) (width 0.5) (layer "F.Cu") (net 13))
 (segment (start 137.922 113.284) (end 136.7536 114.4524) (width 0.5) (layer "F.Cu") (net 13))
 (segment (start 135.5852 115.6208) (end 136.7536 114.4524) (width 0.5) (layer "F.Cu") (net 13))
 (segment (start 137.922 111.5568) (end 137.922 113.284) (width 0.5) (layer "F.Cu") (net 13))
 (segment (start 157.6051 103.7101) (end 157.734 103.5812) (width 0.5) (layer "F.Cu") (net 5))
 (segment (start 155.1432 103.7101) (end 155.1432 101.2933) (width 0.5) (layer "F.Cu") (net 5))
 (segment (start 155.1432 103.7101) (end 157.6051 103.7101) (width 0.5) (layer "F.Cu") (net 5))
 (segment (start 156.9955 103.5812) (end 157.734 103.5812) (width 0.25) (layer "F.Cu") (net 5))
 (segment (start 155.1432 101.2933) (end 155.1686 101.2679) (width 0.5) (layer "F.Cu") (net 5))
 (segment (start 160.8328 103.8352) (end 157.988 103.8352) (width 0.5) (layer "F.Cu") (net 5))
 (segment (start 157.988 103.8352) (end 157.734 103.5812) (width 0.5) (layer "F.Cu") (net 5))
 (segment (start 154.051 106.6273) (end 155.1432 105.5351) (width 0.5) (layer "F.Cu") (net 9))
 (segment (start 154.051 108.0643) (end 154.051 106.6273) (width 0.5) (layer "F.Cu") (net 9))
 (segment (start 151.6634 107.1118) (end 152.9406 108.389) (width 0.5) (layer "F.Cu") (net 10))
 (segment (start 154.0256 116.5606) (end 154.432 116.5606) (width 0.5) (layer "F.Cu") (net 10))
 (segment (start 156.4386 113.4872) (end 154.3812 113.4872) (width 0.5) (layer "F.Cu") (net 10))
 (segment (start 154.3812 116.5098) (end 154.432 116.5606) (width 0.5) (layer "F.Cu") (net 10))
 (segment (start 154.432 116.5606) (end 155.448 116.5606) (width 0.5) (layer "F.Cu") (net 10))
 (segment (start 154.3812 113.4872) (end 154.3812 116.5098) (width 0.5) (layer "F.Cu") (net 10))
 (segment (start 152.9842 117.602) (end 154.0256 116.5606) (width 0.5) (layer "F.Cu") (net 10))
 (segment (start 151.765 117.602) (end 152.9842 117.602) (width 0.5) (layer "F.Cu") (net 10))
 (segment (start 154.3812 111.5822) (end 154.3812 113.4872) (width 0.5) (layer "F.Cu") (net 10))
 (segment (start 152.9406 110.1416) (end 154.3812 111.5822) (width 0.5) (layer "F.Cu") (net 10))
 (segment (start 152.9406 108.389) (end 152.9406 110.1416) (width 0.5) (layer "F.Cu") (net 10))
 (segment (start 166.7256 107.1626) (end 166.7256 103.886) (width 1) (layer "F.Cu") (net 16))
 (segment (start 165.7096 108.1786) (end 166.7256 107.1626) (width 1) (layer "F.Cu") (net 16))
 (segment (start 166.7256 103.886) (end 166.6748 103.8352) (width 1) (layer "F.Cu") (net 16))
 (segment (start 166.6748 103.8352) (end 166.6748 100.0252) (width 1) (layer "F.Cu") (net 16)))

